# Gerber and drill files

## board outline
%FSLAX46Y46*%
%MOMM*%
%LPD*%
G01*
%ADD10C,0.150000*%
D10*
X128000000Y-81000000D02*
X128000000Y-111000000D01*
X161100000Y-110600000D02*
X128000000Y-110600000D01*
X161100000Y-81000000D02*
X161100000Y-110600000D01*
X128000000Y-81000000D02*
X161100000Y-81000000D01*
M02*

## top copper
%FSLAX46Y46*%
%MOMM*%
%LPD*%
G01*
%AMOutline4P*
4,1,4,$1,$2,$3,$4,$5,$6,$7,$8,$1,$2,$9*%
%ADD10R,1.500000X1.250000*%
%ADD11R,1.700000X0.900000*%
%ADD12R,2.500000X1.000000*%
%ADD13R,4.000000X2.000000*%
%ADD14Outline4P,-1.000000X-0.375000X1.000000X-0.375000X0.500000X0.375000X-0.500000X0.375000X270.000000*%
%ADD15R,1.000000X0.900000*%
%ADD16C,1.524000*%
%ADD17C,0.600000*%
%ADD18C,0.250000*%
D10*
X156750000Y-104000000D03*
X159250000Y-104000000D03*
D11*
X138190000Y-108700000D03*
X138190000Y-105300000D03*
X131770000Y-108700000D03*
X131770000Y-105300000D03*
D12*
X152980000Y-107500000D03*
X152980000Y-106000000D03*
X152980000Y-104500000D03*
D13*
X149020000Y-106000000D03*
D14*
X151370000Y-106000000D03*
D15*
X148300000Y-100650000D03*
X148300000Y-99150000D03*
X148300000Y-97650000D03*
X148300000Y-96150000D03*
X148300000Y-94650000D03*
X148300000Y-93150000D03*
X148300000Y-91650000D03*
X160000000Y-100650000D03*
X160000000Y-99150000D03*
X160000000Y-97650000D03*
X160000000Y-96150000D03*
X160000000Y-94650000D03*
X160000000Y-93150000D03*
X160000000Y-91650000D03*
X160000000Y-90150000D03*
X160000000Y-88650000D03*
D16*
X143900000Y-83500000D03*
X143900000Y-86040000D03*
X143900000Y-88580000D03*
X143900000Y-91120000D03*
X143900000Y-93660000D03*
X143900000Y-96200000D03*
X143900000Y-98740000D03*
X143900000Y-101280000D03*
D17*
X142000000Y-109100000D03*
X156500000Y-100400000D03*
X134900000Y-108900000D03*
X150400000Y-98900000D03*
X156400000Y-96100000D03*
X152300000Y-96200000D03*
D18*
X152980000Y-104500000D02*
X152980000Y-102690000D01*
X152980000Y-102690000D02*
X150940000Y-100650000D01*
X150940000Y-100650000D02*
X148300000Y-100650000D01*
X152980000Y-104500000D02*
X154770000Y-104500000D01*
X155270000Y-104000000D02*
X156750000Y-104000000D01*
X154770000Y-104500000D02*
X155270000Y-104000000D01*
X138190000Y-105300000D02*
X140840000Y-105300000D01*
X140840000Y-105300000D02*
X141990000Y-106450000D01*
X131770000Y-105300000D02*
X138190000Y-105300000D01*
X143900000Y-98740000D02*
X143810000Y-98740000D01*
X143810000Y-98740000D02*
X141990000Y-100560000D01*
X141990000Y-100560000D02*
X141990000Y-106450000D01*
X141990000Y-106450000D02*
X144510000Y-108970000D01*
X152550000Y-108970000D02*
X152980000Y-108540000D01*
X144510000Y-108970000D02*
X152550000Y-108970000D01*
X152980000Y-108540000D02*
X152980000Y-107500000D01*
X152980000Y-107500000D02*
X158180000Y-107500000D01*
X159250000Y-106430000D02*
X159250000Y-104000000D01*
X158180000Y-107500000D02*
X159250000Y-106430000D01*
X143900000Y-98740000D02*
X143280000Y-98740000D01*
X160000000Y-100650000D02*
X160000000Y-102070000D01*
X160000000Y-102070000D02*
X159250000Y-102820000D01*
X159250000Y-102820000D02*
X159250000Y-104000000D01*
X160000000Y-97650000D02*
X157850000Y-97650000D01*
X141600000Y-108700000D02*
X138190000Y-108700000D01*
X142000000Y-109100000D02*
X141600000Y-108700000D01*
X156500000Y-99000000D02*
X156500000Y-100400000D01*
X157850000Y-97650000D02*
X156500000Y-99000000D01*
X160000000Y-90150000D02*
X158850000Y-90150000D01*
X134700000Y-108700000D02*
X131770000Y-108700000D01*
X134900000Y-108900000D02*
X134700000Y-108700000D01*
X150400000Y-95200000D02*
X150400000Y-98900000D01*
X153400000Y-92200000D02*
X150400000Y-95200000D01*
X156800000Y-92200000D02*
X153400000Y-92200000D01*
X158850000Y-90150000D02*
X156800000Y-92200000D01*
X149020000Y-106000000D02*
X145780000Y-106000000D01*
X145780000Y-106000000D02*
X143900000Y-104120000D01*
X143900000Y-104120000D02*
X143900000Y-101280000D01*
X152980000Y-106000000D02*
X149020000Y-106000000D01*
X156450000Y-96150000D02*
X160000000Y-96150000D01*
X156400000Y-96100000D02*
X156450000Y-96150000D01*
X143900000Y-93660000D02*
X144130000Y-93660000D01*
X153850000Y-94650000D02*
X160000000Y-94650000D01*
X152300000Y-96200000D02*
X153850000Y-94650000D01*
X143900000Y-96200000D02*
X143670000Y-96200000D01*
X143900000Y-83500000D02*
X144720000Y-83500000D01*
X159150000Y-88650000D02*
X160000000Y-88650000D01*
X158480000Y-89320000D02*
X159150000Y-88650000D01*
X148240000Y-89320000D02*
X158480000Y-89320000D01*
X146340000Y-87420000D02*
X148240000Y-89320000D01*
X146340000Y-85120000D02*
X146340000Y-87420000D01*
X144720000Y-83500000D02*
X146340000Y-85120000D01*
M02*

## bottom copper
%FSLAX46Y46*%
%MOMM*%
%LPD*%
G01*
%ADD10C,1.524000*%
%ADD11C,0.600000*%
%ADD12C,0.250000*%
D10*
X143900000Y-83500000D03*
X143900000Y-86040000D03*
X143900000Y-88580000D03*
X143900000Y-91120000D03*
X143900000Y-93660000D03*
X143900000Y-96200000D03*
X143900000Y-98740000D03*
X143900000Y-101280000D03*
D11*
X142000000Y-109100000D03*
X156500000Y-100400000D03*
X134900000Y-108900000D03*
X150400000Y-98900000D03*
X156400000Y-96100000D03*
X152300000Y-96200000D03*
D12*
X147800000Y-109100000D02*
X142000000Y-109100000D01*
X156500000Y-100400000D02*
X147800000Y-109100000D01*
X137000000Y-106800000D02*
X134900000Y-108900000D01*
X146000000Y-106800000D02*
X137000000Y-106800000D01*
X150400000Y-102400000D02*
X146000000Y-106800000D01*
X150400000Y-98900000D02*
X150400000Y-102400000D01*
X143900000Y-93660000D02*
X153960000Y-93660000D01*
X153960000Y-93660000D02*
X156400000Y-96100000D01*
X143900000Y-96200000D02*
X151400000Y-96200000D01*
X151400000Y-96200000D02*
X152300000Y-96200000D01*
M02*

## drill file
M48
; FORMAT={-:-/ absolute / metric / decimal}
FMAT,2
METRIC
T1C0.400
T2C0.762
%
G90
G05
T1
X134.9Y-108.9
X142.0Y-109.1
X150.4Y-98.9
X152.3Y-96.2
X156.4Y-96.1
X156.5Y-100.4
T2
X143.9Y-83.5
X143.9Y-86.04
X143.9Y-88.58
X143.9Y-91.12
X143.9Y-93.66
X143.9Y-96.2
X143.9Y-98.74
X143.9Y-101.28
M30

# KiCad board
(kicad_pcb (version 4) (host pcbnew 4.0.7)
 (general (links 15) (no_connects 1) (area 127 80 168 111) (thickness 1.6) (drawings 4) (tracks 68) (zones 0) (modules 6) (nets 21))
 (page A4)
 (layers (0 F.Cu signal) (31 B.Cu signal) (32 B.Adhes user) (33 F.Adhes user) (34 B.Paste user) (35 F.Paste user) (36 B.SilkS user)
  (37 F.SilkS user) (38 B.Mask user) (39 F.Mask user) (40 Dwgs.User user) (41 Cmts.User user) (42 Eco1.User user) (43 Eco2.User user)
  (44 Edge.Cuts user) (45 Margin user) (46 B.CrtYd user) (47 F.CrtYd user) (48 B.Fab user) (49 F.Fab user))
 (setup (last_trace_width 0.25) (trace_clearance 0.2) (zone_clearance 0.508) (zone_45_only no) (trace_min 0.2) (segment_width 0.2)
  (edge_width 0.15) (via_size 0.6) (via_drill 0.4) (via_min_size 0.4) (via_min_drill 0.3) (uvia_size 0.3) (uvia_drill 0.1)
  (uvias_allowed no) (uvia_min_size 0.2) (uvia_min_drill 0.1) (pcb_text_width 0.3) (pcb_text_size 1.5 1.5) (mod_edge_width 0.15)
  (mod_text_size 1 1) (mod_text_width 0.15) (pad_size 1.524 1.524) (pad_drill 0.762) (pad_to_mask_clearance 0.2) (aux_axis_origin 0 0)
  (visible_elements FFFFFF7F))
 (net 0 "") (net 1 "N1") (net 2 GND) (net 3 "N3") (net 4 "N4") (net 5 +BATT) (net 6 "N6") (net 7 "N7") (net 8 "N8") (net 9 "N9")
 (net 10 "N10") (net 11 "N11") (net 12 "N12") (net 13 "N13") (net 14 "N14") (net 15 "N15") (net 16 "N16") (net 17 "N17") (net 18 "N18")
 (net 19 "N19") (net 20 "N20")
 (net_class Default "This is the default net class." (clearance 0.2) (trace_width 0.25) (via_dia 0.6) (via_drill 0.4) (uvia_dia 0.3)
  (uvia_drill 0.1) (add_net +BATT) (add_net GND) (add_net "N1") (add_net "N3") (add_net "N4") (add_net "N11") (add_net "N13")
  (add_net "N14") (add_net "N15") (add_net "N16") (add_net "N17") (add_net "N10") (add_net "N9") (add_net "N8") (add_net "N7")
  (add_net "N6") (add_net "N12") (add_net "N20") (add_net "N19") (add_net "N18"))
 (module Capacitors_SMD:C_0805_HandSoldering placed (layer F.Cu) (at 158 104)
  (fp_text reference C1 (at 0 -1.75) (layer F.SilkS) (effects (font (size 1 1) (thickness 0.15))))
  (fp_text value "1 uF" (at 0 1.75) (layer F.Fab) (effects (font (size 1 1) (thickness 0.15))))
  (pad 1 smd rect (at -1.25 0) (size 1.5 1.25) (layers F.Cu F.Paste F.Mask) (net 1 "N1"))
  (pad 2 smd rect (at 1.25 0) (size 1.5 1.25) (layers F.Cu F.Paste F.Mask) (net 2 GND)))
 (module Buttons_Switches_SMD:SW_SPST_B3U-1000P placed (layer F.Cu) (at 138.19 107 90)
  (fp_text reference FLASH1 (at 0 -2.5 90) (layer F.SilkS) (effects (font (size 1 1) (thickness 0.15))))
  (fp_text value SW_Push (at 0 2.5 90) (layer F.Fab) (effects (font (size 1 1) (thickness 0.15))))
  (pad 1 smd rect (at -1.7 0 90) (size 0.9 1.7) (layers F.Cu F.Paste F.Mask) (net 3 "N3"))
  (pad 2 smd rect (at 1.7 0 90) (size 0.9 1.7) (layers F.Cu F.Paste F.Mask) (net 2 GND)))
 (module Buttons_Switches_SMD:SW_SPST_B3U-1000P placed (layer F.Cu) (at 131.77 107 90)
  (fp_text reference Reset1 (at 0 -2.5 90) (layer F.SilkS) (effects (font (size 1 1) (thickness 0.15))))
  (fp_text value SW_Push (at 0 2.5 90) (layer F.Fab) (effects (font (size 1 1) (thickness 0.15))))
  (pad 1 smd rect (at -1.7 0 90) (size 0.9 1.7) (layers F.Cu F.Paste F.Mask) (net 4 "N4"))
  (pad 2 smd rect (at 1.7 0 90) (size 0.9 1.7) (layers F.Cu F.Paste F.Mask) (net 2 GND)))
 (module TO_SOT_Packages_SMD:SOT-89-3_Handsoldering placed (layer F.Cu) (at 151 106 180)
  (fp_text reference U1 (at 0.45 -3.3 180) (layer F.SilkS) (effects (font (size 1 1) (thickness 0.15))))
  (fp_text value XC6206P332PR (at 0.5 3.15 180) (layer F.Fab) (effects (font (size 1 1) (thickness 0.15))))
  (pad 1 smd rect (at -1.98 -1.5 90) (size 1 2.5) (layers F.Cu F.Paste F.Mask) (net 2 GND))
  (pad 2 smd rect (at -1.98 0 90) (size 1 2.5) (layers F.Cu F.Paste F.Mask) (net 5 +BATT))
  (pad 3 smd rect (at -1.98 1.5 90) (size 1 2.5) (layers F.Cu F.Paste F.Mask) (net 1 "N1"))
  (pad 2 smd rect (at 1.98 0 90) (size 2 4) (layers F.Cu F.Paste F.Mask) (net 5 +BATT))
  (pad 2 smd trapezoid (at -0.37 0 270) (size 1.5 0.75) (rect_delta 0 0.5) (layers F.Cu F.Paste F.Mask) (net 5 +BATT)))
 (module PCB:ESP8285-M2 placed (layer F.Cu) (at 148 102)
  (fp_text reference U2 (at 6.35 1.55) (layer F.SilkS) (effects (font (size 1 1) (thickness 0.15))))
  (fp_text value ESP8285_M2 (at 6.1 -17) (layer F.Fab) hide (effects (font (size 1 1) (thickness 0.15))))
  (pad 7 smd rect (at 0.3 -1.35) (size 1 0.9) (layers F.Cu F.Paste F.Mask) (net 1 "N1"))
  (pad 6 smd rect (at 0.3 -2.85) (size 1 0.9) (layers F.Cu F.Paste F.Mask) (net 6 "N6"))
  (pad 5 smd rect (at 0.3 -4.35) (size 1 0.9) (layers F.Cu F.Paste F.Mask) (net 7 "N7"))
  (pad 4 smd rect (at 0.3 -5.85) (size 1 0.9) (layers F.Cu F.Paste F.Mask) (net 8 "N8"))
  (pad 3 smd rect (at 0.3 -7.35) (size 1 0.9) (layers F.Cu F.Paste F.Mask) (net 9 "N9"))
  (pad 2 smd rect (at 0.3 -8.85) (size 1 0.9) (layers F.Cu F.Paste F.Mask) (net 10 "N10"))
  (pad 1 smd rect (at 0.3 -10.35) (size 1 0.9) (layers F.Cu F.Paste F.Mask) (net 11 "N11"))
  (pad 8 smd rect (at 12 -1.35) (size 1 0.9) (layers F.Cu F.Paste F.Mask) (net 2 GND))
  (pad 9 smd rect (at 12 -2.85) (size 1 0.9) (layers F.Cu F.Paste F.Mask) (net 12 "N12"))
  (pad 10 smd rect (at 12 -4.35) (size 1 0.9) (layers F.Cu F.Paste F.Mask) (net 3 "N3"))
  (pad 11 smd rect (at 12 -5.85) (size 1 0.9) (layers F.Cu F.Paste F.Mask) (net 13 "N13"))
  (pad 12 smd rect (at 12 -7.35) (size 1 0.9) (layers F.Cu F.Paste F.Mask) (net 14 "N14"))
  (pad 13 smd rect (at 12 -8.85) (size 1 0.9) (layers F.Cu F.Paste F.Mask) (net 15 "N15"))
  (pad 14 smd rect (at 12 -10.35) (size 1 0.9) (layers F.Cu F.Paste F.Mask) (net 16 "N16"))
  (pad 15 smd rect (at 12 -11.85) (size 1 0.9) (layers F.Cu F.Paste F.Mask) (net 4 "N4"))
  (pad 16 smd rect (at 12 -13.35) (size 1 0.9) (layers F.Cu F.Paste F.Mask) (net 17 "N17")))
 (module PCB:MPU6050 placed (layer F.Cu) (at 145 82 180)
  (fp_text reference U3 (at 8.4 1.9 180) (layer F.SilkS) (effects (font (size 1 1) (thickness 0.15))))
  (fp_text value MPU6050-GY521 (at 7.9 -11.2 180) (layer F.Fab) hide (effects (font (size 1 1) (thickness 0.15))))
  (pad 8 thru_hole circle (at 1.1 -1.5 180) (size 1.524 1.524) (drill 0.762) (layers *.Cu *.Mask) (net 17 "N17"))
  (pad 7 thru_hole circle (at 1.1 -4.04 180) (size 1.524 1.524) (drill 0.762) (layers *.Cu *.Mask) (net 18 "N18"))
  (pad 6 thru_hole circle (at 1.1 -6.58 180) (size 1.524 1.524) (drill 0.762) (layers *.Cu *.Mask) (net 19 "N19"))
  (pad 5 thru_hole circle (at 1.1 -9.12 180) (size 1.524 1.524) (drill 0.762) (layers *.Cu *.Mask) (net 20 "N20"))
  (pad 4 thru_hole circle (at 1.1 -11.66 180) (size 1.524 1.524) (drill 0.762) (layers *.Cu *.Mask) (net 13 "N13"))
  (pad 3 thru_hole circle (at 1.1 -14.2 180) (size 1.524 1.524) (drill 0.762) (layers *.Cu *.Mask) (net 14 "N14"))
  (pad 2 thru_hole circle (at 1.1 -16.74 180) (size 1.524 1.524) (drill 0.762) (layers *.Cu *.Mask) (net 2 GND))
  (pad 1 thru_hole circle (at 1.1 -19.28 180) (size 1.524 1.524) (drill 0.762) (layers *.Cu *.Mask) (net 5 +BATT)))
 (gr_line (start 128 81) (end 128 111) (angle 90) (layer Edge.Cuts) (width 0.15))
 (gr_line (start 161.1 110.6) (end 128 110.6) (angle 90) (layer Edge.Cuts) (width 0.15))
 (gr_line (start 161.1 81) (end 161.1 110.6) (angle 90) (layer Edge.Cuts) (width 0.15))
 (gr_line (start 128 81) (end 161.1 81) (angle 90) (layer Edge.Cuts) (width 0.15))
 (segment (start 152.98 104.5) (end 152.98 102.69) (width 0.25) (layer F.Cu) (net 1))
 (segment (start 152.98 102.69) (end 150.94 100.65) (width 0.25) (layer F.Cu) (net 1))
 (segment (start 150.94 100.65) (end 148.3 100.65) (width 0.25) (layer F.Cu) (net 1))
 (segment (start 152.98 104.5) (end 154.77 104.5) (width 0.25) (layer F.Cu) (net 1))
 (segment (start 155.27 104) (end 156.75 104) (width 0.25) (layer F.Cu) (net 1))
 (segment (start 154.77 104.5) (end 155.27 104) (width 0.25) (layer F.Cu) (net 1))
 (segment (start 138.19 105.3) (end 140.84 105.3) (width 0.25) (layer F.Cu) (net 2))
 (segment (start 140.84 105.3) (end 141.99 106.45) (width 0.25) (layer F.Cu) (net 2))
 (segment (start 131.77 105.3) (end 138.19 105.3) (width 0.25) (layer F.Cu) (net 2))
 (segment (start 143.9 98.74) (end 143.81 98.74) (width 0.25) (layer F.Cu) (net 2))
 (segment (start 143.81 98.74) (end 141.99 100.56) (width 0.25) (layer F.Cu) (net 2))
 (segment (start 141.99 100.56) (end 141.99 106.45) (width 0.25) (layer F.Cu) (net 2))
 (segment (start 141.99 106.45) (end 144.51 108.97) (width 0.25) (layer F.Cu) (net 2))
 (segment (start 152.55 108.97) (end 152.98 108.54) (width 0.25) (layer F.Cu) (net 2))
 (segment (start 144.51 108.97) (end 152.55 108.97) (width 0.25) (layer F.Cu) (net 2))
 (segment (start 152.98 108.54) (end 152.98 107.5) (width 0.25) (layer F.Cu) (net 2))
 (segment (start 152.98 107.5) (end 158.18 107.5) (width 0.25) (layer F.Cu) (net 2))
 (segment (start 159.25 106.43) (end 159.25 104) (width 0.25) (layer F.Cu) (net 2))
 (segment (start 158.18 107.5) (end 159.25 106.43) (width 0.25) (layer F.Cu) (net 2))
 (segment (start 143.9 98.74) (end 143.28 98.74) (width 0.25) (layer F.Cu) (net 2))
 (segment (start 160 100.65) (end 160 102.07) (width 0.25) (layer F.Cu) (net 2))
 (segment (start 160 102.07) (end 159.25 102.82) (width 0.25) (layer F.Cu) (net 2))
 (segment (start 159.25 102.82) (end 159.25 104) (width 0.25) (layer F.Cu) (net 2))
 (segment (start 160 97.65) (end 157.85 97.65) (width 0.25) (layer F.Cu) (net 3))
 (segment (start 141.6 108.7) (end 138.19 108.7) (width 0.25) (layer F.Cu) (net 3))
 (segment (start 142 109.1) (end 141.6 108.7) (width 0.25) (layer F.Cu) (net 3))
 (via (at 142 109.1) (size 0.6) (drill 0.4) (layers F.Cu B.Cu) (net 3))
 (segment (start 147.8 109.1) (end 142 109.1) (width 0.25) (layer B.Cu) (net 3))
 (segment (start 156.5 100.4) (end 147.8 109.1) (width 0.25) (layer B.Cu) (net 3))
 (via (at 156.5 100.4) (size 0.6) (drill 0.4) (layers F.Cu B.Cu) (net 3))
 (segment (start 156.5 99) (end 156.5 100.4) (width 0.25) (layer F.Cu) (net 3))
 (segment (start 157.85 97.65) (end 156.5 99) (width 0.25) (layer F.Cu) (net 3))
 (segment (start 160 90.15) (end 158.85 90.15) (width 0.25) (layer F.Cu) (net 4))
 (segment (start 134.7 108.7) (end 131.77 108.7) (width 0.25) (layer F.Cu) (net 4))
 (segment (start 134.9 108.9) (end 134.7 108.7) (width 0.25) (layer F.Cu) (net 4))
 (via (at 134.9 108.9) (size 0.6) (drill 0.4) (layers F.Cu B.Cu) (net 4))
 (segment (start 137 106.8) (end 134.9 108.9) (width 0.25) (layer B.Cu) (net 4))
 (segment (start 146 106.8) (end 137 106.8) (width 0.25) (layer B.Cu) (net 4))
 (segment (start 150.4 102.4) (end 146 106.8) (width 0.25) (layer B.Cu) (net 4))
 (segment (start 150.4 98.9) (end 150.4 102.4) (width 0.25) (layer B.Cu) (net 4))
 (via (at 150.4 98.9) (size 0.6) (drill 0.4) (layers F.Cu B.Cu) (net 4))
 (segment (start 150.4 95.2) (end 150.4 98.9) (width 0.25) (layer F.Cu) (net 4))
 (segment (start 153.4 92.2) (end 150.4 95.2) (width 0.25) (layer F.Cu) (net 4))
 (segment (start 156.8 92.2) (end 153.4 92.2) (width 0.25) (layer F.Cu) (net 4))
 (segment (start 158.85 90.15) (end 156.8 92.2) (width 0.25) (layer F.Cu) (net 4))
 (segment (start 149.02 106) (end 145.78 106) (width 0.25) (layer F.Cu) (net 5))
 (segment (start 145.78 106) (end 143.9 104.12) (width 0.25) (layer F.Cu) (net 5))
 (segment (start 143.9 104.12) (end 143.9 101.28) (width 0.25) (layer F.Cu) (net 5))
 (segment (start 152.98 106) (end 149.02 106) (width 0.25) (layer F.Cu) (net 5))
 (segment (start 143.9 93.66) (end 153.96 93.66) (width 0.25) (layer B.Cu) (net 13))
 (segment (start 156.45 96.15) (end 160 96.15) (width 0.25) (layer F.Cu) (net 13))
 (segment (start 156.4 96.1) (end 156.45 96.15) (width 0.25) (layer F.Cu) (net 13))
 (via (at 156.4 96.1) (size 0.6) (drill 0.4) (layers F.Cu B.Cu) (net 13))
 (segment (start 153.96 93.66) (end 156.4 96.1) (width 0.25) (layer B.Cu) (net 13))
 (segment (start 143.9 93.66) (end 144.13 93.66) (width 0.25) (layer F.Cu) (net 13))
 (segment (start 143.9 96.2) (end 151.4 96.2) (width 0.25) (layer B.Cu) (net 14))
 (segment (start 153.85 94.65) (end 160 94.65) (width 0.25) (layer F.Cu) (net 14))
 (segment (start 152.3 96.2) (end 153.85 94.65) (width 0.25) (layer F.Cu) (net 14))
 (via (at 152.3 96.2) (size 0.6) (drill 0.4) (layers F.Cu B.Cu) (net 14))
 (segment (start 151.4 96.2) (end 152.3 96.2) (width 0.25) (layer B.Cu) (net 14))
 (segment (start 143.9 96.2) (end 143.67 96.2) (width 0.25) (layer F.Cu) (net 14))
 (segment (start 143.9 83.5) (end 144.72 83.5) (width 0.25) (layer F.Cu) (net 17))
 (segment (start 159.15 88.65) (end 160 88.65) (width 0.25) (layer F.Cu) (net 17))
 (segment (start 158.48 89.32) (end 159.15 88.65) (width 0.25) (layer F.Cu) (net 17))
 (segment (start 148.24 89.32) (end 158.48 89.32) (width 0.25) (layer F.Cu) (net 17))
 (segment (start 146.34 87.42) (end 148.24 89.32) (width 0.25) (layer F.Cu) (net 17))
 (segment (start 146.34 85.12) (end 146.34 87.42) (width 0.25) (layer F.Cu) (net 17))
 (segment (start 144.72 83.5) (end 146.34 85.12) (width 0.25) (layer F.Cu) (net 17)))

